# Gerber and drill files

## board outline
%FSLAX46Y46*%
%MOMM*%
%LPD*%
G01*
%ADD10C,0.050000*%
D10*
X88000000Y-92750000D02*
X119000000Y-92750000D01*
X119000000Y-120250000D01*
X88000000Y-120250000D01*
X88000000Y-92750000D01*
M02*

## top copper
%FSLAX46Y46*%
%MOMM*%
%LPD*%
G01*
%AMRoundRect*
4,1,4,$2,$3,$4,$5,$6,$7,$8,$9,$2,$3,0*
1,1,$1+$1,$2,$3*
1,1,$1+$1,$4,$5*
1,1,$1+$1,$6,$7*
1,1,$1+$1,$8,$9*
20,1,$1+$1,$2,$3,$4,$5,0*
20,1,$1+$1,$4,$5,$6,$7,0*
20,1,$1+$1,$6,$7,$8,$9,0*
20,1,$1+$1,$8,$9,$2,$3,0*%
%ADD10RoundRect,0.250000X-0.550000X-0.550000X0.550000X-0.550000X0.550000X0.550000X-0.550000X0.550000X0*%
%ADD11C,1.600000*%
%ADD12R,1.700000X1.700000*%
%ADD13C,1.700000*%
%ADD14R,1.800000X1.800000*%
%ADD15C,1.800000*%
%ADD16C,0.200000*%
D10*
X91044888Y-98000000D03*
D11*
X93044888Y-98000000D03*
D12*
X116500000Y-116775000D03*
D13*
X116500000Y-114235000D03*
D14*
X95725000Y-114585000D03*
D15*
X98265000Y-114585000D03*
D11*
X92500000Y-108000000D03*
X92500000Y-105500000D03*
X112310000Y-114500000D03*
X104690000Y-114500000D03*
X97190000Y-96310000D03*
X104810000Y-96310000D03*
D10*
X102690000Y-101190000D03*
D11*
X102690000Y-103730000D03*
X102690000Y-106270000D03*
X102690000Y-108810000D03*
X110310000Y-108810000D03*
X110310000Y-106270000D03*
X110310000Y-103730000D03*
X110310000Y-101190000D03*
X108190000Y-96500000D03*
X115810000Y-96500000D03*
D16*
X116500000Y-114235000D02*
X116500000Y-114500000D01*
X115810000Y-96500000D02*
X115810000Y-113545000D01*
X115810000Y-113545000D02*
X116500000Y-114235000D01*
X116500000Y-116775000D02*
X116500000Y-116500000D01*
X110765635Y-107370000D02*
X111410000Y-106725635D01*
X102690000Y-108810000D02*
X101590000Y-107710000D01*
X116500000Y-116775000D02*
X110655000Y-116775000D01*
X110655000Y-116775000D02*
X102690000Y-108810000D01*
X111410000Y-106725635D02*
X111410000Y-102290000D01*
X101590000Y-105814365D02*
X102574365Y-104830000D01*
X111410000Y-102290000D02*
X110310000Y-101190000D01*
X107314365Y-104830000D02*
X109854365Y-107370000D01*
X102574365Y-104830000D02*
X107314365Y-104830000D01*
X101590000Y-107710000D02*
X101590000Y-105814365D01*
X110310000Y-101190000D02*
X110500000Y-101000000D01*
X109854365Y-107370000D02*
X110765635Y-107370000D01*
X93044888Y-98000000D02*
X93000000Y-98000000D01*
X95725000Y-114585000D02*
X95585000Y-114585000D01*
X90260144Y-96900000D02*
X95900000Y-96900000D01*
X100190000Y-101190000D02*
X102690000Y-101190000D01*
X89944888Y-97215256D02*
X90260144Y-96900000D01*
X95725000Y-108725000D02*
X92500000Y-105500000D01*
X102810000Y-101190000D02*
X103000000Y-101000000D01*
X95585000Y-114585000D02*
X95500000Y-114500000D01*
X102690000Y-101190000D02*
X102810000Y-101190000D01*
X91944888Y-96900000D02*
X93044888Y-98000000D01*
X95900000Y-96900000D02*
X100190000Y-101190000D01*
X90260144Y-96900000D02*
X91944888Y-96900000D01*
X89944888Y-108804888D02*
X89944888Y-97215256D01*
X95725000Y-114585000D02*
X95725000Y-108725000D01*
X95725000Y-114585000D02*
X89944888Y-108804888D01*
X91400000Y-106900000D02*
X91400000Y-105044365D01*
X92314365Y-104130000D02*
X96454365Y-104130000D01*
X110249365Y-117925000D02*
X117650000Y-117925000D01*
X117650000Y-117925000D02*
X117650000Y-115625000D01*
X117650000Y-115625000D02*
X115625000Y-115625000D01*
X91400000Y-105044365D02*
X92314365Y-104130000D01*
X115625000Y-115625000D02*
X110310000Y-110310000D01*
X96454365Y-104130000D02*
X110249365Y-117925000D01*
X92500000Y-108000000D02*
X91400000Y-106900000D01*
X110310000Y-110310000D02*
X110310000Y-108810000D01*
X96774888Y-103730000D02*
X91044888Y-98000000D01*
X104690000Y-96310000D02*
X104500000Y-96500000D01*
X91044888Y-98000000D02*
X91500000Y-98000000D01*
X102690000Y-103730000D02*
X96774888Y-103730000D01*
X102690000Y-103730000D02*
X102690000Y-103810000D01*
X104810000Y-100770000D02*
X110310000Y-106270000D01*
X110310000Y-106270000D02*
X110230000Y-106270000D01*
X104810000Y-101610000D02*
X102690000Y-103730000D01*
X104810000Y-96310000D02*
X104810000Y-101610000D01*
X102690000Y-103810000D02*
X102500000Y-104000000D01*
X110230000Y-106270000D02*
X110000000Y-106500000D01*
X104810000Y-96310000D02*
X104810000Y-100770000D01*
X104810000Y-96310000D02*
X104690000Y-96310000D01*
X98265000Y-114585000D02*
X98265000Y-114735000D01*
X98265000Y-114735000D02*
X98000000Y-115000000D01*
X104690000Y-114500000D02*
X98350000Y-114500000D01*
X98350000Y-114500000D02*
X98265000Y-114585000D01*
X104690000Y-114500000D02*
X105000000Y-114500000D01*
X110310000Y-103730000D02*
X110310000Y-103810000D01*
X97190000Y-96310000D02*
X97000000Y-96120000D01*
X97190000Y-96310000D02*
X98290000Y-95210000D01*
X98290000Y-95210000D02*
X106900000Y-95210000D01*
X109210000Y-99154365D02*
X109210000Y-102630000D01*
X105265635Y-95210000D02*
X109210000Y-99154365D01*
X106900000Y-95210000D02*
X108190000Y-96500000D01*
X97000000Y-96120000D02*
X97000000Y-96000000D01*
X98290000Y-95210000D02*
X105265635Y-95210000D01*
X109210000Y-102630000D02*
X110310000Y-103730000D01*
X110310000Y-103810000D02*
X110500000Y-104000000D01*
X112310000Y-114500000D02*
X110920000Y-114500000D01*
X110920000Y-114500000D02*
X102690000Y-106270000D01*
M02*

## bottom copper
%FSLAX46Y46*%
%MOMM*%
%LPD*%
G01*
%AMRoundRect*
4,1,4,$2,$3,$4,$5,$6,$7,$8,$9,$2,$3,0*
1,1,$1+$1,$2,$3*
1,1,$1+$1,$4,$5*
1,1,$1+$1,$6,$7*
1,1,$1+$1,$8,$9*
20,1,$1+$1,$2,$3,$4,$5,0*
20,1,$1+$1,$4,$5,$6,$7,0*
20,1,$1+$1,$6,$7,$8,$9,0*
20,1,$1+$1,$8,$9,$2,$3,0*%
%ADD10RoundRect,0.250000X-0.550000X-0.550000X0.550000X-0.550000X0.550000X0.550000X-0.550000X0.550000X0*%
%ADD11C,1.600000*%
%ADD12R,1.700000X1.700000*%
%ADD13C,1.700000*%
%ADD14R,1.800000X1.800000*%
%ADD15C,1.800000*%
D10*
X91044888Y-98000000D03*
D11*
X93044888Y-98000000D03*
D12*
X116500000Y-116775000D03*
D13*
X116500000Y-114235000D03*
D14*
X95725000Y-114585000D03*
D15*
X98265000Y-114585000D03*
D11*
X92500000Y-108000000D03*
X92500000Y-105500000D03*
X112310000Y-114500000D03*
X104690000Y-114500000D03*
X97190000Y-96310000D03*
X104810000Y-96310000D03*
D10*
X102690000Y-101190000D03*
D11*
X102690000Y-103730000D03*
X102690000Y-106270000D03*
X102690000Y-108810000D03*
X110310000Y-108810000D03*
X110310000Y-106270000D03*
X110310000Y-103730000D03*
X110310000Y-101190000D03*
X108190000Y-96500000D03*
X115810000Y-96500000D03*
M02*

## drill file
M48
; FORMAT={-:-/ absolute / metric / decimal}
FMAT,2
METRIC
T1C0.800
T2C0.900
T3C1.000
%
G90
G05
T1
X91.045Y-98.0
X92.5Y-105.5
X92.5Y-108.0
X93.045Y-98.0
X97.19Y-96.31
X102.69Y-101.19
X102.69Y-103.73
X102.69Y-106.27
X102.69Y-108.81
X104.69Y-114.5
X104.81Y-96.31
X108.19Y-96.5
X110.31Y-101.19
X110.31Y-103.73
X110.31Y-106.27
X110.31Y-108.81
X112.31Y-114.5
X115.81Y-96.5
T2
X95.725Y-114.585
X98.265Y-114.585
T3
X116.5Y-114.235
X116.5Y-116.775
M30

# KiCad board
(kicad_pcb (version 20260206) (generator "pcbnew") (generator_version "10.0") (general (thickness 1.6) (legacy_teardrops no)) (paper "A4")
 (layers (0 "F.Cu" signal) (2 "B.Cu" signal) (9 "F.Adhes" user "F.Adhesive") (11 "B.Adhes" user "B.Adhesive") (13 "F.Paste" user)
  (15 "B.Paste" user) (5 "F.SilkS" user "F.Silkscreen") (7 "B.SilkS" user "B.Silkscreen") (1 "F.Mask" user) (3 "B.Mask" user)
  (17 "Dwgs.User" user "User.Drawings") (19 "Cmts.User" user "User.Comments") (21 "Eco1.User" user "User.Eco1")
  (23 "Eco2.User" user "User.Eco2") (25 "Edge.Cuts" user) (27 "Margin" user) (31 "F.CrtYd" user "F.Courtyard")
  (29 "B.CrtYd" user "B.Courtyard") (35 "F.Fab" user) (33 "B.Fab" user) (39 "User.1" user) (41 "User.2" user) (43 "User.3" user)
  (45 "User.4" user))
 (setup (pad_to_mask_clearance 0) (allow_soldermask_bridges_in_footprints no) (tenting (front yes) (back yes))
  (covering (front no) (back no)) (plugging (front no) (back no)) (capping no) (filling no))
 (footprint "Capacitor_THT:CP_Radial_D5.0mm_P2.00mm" (layer "F.Cu") (at 91.044888 98)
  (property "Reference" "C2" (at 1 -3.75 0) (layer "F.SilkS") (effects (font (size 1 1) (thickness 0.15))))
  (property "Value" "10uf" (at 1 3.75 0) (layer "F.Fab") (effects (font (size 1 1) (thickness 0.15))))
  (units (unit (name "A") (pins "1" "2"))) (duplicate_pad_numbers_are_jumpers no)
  (pad "1" thru_hole roundrect (at 0 0) (size 1.6 1.6) (drill 0.8) (layers "*.Cu" "*.Mask") (remove_unused_layers no)
   (roundrect_rratio 0.15625) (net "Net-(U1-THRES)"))
  (pad "2" thru_hole circle (at 2 0) (size 1.6 1.6) (drill 0.8) (layers "*.Cu" "*.Mask") (remove_unused_layers no) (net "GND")))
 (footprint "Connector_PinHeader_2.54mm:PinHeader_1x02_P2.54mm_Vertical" (layer "F.Cu") (at 116.5 116.775 180)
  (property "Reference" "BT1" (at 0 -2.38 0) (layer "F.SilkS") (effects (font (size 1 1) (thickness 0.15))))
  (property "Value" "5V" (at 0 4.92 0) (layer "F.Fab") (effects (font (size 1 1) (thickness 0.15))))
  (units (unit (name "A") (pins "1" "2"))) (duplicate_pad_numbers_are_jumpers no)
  (pad "1" thru_hole rect (at 0 0 180) (size 1.7 1.7) (drill 1) (layers "*.Cu" "*.Mask") (remove_unused_layers no) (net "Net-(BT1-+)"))
  (pad "2" thru_hole circle (at 0 2.54 180) (size 1.7 1.7) (drill 1) (layers "*.Cu" "*.Mask") (remove_unused_layers no) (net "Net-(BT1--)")))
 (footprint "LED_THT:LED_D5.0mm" (layer "F.Cu") (at 95.725 114.585)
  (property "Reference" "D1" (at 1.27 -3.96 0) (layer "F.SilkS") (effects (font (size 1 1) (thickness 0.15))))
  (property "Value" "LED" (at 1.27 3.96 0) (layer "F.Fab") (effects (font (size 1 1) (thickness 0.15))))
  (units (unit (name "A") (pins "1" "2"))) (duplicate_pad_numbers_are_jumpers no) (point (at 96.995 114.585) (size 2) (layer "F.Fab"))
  (pad "1" thru_hole rect (at 0 0) (size 1.8 1.8) (drill 0.9) (layers "*.Cu" "*.Mask") (remove_unused_layers no) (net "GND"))
  (pad "2" thru_hole circle (at 2.54 0) (size 1.8 1.8) (drill 0.9) (layers "*.Cu" "*.Mask") (remove_unused_layers no) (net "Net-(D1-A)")))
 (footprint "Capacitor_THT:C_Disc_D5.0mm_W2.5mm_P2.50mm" (layer "F.Cu") (at 92.5 108 90)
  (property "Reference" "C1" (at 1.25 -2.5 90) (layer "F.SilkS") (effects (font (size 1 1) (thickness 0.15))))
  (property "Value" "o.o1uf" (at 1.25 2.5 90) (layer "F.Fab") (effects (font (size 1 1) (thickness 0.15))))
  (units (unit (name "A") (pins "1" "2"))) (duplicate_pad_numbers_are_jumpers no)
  (pad "1" thru_hole circle (at 0 0 90) (size 1.6 1.6) (drill 0.8) (layers "*.Cu" "*.Mask") (remove_unused_layers no) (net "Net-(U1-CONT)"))
  (pad "2" thru_hole circle (at 2.5 0 90) (size 1.6 1.6) (drill 0.8) (layers "*.Cu" "*.Mask") (remove_unused_layers no) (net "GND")))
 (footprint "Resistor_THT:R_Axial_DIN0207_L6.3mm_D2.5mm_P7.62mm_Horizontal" (layer "F.Cu") (at 112.31 114.5 180)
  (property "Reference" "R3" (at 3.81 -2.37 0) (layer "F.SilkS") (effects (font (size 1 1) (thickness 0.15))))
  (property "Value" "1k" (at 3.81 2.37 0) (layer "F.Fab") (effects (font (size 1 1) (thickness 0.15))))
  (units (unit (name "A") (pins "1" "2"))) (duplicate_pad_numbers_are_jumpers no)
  (pad "1" thru_hole circle (at 0 0 180) (size 1.6 1.6) (drill 0.8) (layers "*.Cu" "*.Mask") (remove_unused_layers no) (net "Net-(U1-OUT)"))
  (pad "2" thru_hole circle (at 7.62 0 180) (size 1.6 1.6) (drill 0.8) (layers "*.Cu" "*.Mask") (remove_unused_layers no) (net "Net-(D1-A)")))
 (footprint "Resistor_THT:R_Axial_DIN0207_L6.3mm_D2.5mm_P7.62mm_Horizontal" (layer "F.Cu") (at 97.19 96.31)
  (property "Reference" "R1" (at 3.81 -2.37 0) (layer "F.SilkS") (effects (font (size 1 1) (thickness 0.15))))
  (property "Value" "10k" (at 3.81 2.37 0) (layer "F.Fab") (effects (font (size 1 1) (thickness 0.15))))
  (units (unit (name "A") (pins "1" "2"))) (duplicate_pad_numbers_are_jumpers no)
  (pad "1" thru_hole circle (at 0 0) (size 1.6 1.6) (drill 0.8) (layers "*.Cu" "*.Mask") (remove_unused_layers no) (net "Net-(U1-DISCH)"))
  (pad "2" thru_hole circle (at 7.62 0) (size 1.6 1.6) (drill 0.8) (layers "*.Cu" "*.Mask") (remove_unused_layers no) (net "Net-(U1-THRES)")))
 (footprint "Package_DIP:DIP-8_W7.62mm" (layer "F.Cu") (at 102.69 101.19)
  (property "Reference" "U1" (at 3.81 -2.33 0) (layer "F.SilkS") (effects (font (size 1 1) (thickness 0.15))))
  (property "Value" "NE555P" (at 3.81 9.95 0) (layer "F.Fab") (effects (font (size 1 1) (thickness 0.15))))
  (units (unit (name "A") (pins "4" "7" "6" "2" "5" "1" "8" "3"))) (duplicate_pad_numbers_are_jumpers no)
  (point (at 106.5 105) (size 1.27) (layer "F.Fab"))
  (pad "1" thru_hole roundrect (at 0 0) (size 1.6 1.6) (drill 0.8) (layers "*.Cu" "*.Mask") (remove_unused_layers no)
   (roundrect_rratio 0.15625) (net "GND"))
  (pad "2" thru_hole circle (at 0 2.54) (size 1.6 1.6) (drill 0.8) (layers "*.Cu" "*.Mask") (remove_unused_layers no) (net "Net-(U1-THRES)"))
  (pad "3" thru_hole circle (at 0 5.08) (size 1.6 1.6) (drill 0.8) (layers "*.Cu" "*.Mask") (remove_unused_layers no) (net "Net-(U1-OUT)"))
  (pad "4" thru_hole circle (at 0 7.62) (size 1.6 1.6) (drill 0.8) (layers "*.Cu" "*.Mask") (remove_unused_layers no) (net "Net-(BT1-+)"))
  (pad "5" thru_hole circle (at 7.62 7.62) (size 1.6 1.6) (drill 0.8) (layers "*.Cu" "*.Mask") (remove_unused_layers no)
   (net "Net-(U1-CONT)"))
  (pad "6" thru_hole circle (at 7.62 5.08) (size 1.6 1.6) (drill 0.8) (layers "*.Cu" "*.Mask") (remove_unused_layers no)
   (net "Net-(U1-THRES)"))
  (pad "7" thru_hole circle (at 7.62 2.54) (size 1.6 1.6) (drill 0.8) (layers "*.Cu" "*.Mask") (remove_unused_layers no)
   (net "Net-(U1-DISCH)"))
  (pad "8" thru_hole circle (at 7.62 0) (size 1.6 1.6) (drill 0.8) (layers "*.Cu" "*.Mask") (remove_unused_layers no) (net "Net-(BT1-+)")))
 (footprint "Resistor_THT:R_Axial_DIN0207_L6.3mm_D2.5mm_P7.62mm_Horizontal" (layer "F.Cu") (at 108.19 96.5)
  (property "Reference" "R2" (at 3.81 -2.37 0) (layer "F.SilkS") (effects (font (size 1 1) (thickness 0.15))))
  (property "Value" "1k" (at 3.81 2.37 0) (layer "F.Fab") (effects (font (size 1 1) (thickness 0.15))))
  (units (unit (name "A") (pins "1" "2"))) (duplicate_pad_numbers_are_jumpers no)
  (pad "1" thru_hole circle (at 0 0) (size 1.6 1.6) (drill 0.8) (layers "*.Cu" "*.Mask") (remove_unused_layers no) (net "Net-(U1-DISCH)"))
  (pad "2" thru_hole circle (at 7.62 0) (size 1.6 1.6) (drill 0.8) (layers "*.Cu" "*.Mask") (remove_unused_layers no) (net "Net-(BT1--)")))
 (gr_rect (start 88 92.75) (end 119 120.25) (stroke (width 0.05) (type default)) (fill no) (layer "Edge.Cuts"))
 (segment (start 116.5 114.235) (end 116.5 114.5) (width 0.2) (layer "F.Cu") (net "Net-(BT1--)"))
 (segment (start 115.81 96.5) (end 115.81 113.545) (width 0.2) (layer "F.Cu") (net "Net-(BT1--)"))
 (segment (start 115.81 113.545) (end 116.5 114.235) (width 0.2) (layer "F.Cu") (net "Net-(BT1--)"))
 (segment (start 116.5 116.775) (end 116.5 116.5) (width 0.2) (layer "F.Cu") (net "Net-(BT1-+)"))
 (segment (start 110.765635 107.37) (end 111.41 106.725635) (width 0.2) (layer "F.Cu") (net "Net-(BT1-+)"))
 (segment (start 102.69 108.81) (end 101.59 107.71) (width 0.2) (layer "F.Cu") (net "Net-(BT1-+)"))
 (segment (start 116.5 116.775) (end 110.655 116.775) (width 0.2) (layer "F.Cu") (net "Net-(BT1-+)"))
 (segment (start 110.655 116.775) (end 102.69 108.81) (width 0.2) (layer "F.Cu") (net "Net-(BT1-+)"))
 (segment (start 111.41 106.725635) (end 111.41 102.29) (width 0.2) (layer "F.Cu") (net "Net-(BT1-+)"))
 (segment (start 101.59 105.814365) (end 102.574365 104.83) (width 0.2) (layer "F.Cu") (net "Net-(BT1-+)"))
 (segment (start 111.41 102.29) (end 110.31 101.19) (width 0.2) (layer "F.Cu") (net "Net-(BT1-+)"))
 (segment (start 107.314365 104.83) (end 109.854365 107.37) (width 0.2) (layer "F.Cu") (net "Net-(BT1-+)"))
 (segment (start 102.574365 104.83) (end 107.314365 104.83) (width 0.2) (layer "F.Cu") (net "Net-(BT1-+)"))
 (segment (start 101.59 107.71) (end 101.59 105.814365) (width 0.2) (layer "F.Cu") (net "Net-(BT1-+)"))
 (segment (start 110.31 101.19) (end 110.5 101) (width 0.2) (layer "F.Cu") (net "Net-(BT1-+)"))
 (segment (start 109.854365 107.37) (end 110.765635 107.37) (width 0.2) (layer "F.Cu") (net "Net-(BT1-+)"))
 (segment (start 93.044888 98) (end 93 98) (width 0.2) (layer "F.Cu") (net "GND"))
 (segment (start 95.725 114.585) (end 95.585 114.585) (width 0.2) (layer "F.Cu") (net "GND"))
 (segment (start 90.260144 96.9) (end 95.9 96.9) (width 0.2) (layer "F.Cu") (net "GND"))
 (segment (start 100.19 101.19) (end 102.69 101.19) (width 0.2) (layer "F.Cu") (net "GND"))
 (segment (start 89.944888 97.215256) (end 90.260144 96.9) (width 0.2) (layer "F.Cu") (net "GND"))
 (segment (start 95.725 108.725) (end 92.5 105.5) (width 0.2) (layer "F.Cu") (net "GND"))
 (segment (start 102.81 101.19) (end 103 101) (width 0.2) (layer "F.Cu") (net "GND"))
 (segment (start 95.585 114.585) (end 95.5 114.5) (width 0.2) (layer "F.Cu") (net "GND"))
 (segment (start 102.69 101.19) (end 102.81 101.19) (width 0.2) (layer "F.Cu") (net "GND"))
 (segment (start 91.944888 96.9) (end 93.044888 98) (width 0.2) (layer "F.Cu") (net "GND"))
 (segment (start 95.9 96.9) (end 100.19 101.19) (width 0.2) (layer "F.Cu") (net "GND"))
 (segment (start 90.260144 96.9) (end 91.944888 96.9) (width 0.2) (layer "F.Cu") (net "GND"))
 (segment (start 89.944888 108.804888) (end 89.944888 97.215256) (width 0.2) (layer "F.Cu") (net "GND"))
 (segment (start 95.725 114.585) (end 95.725 108.725) (width 0.2) (layer "F.Cu") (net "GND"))
 (segment (start 95.725 114.585) (end 89.944888 108.804888) (width 0.2) (layer "F.Cu") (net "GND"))
 (segment (start 91.4 106.9) (end 91.4 105.044365) (width 0.2) (layer "F.Cu") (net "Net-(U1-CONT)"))
 (segment (start 92.314365 104.13) (end 96.454365 104.13) (width 0.2) (layer "F.Cu") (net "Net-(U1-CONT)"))
 (segment (start 110.249365 117.925) (end 117.65 117.925) (width 0.2) (layer "F.Cu") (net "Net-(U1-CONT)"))
 (segment (start 117.65 117.925) (end 117.65 115.625) (width 0.2) (layer "F.Cu") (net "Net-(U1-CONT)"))
 (segment (start 117.65 115.625) (end 115.625 115.625) (width 0.2) (layer "F.Cu") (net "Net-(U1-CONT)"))
 (segment (start 91.4 105.044365) (end 92.314365 104.13) (width 0.2) (layer "F.Cu") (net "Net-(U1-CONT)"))
 (segment (start 115.625 115.625) (end 110.31 110.31) (width 0.2) (layer "F.Cu") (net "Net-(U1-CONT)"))
 (segment (start 96.454365 104.13) (end 110.249365 117.925) (width 0.2) (layer "F.Cu") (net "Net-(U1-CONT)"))
 (segment (start 92.5 108) (end 91.4 106.9) (width 0.2) (layer "F.Cu") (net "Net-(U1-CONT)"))
 (segment (start 110.31 110.31) (end 110.31 108.81) (width 0.2) (layer "F.Cu") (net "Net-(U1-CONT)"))
 (segment (start 96.774888 103.73) (end 91.044888 98) (width 0.2) (layer "F.Cu") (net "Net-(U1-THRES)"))
 (segment (start 104.69 96.31) (end 104.5 96.5) (width 0.2) (layer "F.Cu") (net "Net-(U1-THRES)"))
 (segment (start 91.044888 98) (end 91.5 98) (width 0.2) (layer "F.Cu") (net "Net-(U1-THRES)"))
 (segment (start 102.69 103.73) (end 96.774888 103.73) (width 0.2) (layer "F.Cu") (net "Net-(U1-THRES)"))
 (segment (start 102.69 103.73) (end 102.69 103.81) (width 0.2) (layer "F.Cu") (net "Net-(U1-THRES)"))
 (segment (start 104.81 100.77) (end 110.31 106.27) (width 0.2) (layer "F.Cu") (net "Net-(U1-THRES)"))
 (segment (start 110.31 106.27) (end 110.23 106.27) (width 0.2) (layer "F.Cu") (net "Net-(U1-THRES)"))
 (segment (start 104.81 101.61) (end 102.69 103.73) (width 0.2) (layer "F.Cu") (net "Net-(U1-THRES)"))
 (segment (start 104.81 96.31) (end 104.81 101.61) (width 0.2) (layer "F.Cu") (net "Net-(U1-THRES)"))
 (segment (start 102.69 103.81) (end 102.5 104) (width 0.2) (layer "F.Cu") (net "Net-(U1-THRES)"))
 (segment (start 110.23 106.27) (end 110 106.5) (width 0.2) (layer "F.Cu") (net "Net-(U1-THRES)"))
 (segment (start 104.81 96.31) (end 104.81 100.77) (width 0.2) (layer "F.Cu") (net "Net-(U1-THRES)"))
 (segment (start 104.81 96.31) (end 104.69 96.31) (width 0.2) (layer "F.Cu") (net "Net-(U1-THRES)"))
 (segment (start 98.265 114.585) (end 98.265 114.735) (width 0.2) (layer "F.Cu") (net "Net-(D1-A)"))
 (segment (start 98.265 114.735) (end 98 115) (width 0.2) (layer "F.Cu") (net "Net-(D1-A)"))
 (segment (start 104.69 114.5) (end 98.35 114.5) (width 0.2) (layer "F.Cu") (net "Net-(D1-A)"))
 (segment (start 98.35 114.5) (end 98.265 114.585) (width 0.2) (layer "F.Cu") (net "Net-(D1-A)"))
 (segment (start 104.69 114.5) (end 105 114.5) (width 0.2) (layer "F.Cu") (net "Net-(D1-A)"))
 (segment (start 110.31 103.73) (end 110.31 103.81) (width 0.2) (layer "F.Cu") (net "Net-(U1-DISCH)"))
 (segment (start 97.19 96.31) (end 97 96.12) (width 0.2) (layer "F.Cu") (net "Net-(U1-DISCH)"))
 (segment (start 97.19 96.31) (end 98.29 95.21) (width 0.2) (layer "F.Cu") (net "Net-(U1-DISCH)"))
 (segment (start 98.29 95.21) (end 106.9 95.21) (width 0.2) (layer "F.Cu") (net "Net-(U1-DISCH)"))
 (segment (start 109.21 99.154365) (end 109.21 102.63) (width 0.2) (layer "F.Cu") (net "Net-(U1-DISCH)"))
 (segment (start 105.265635 95.21) (end 109.21 99.154365) (width 0.2) (layer "F.Cu") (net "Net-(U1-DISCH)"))
 (segment (start 106.9 95.21) (end 108.19 96.5) (width 0.2) (layer "F.Cu") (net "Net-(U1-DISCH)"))
 (segment (start 97 96.12) (end 97 96) (width 0.2) (layer "F.Cu") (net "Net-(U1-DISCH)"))
 (segment (start 98.29 95.21) (end 105.265635 95.21) (width 0.2) (layer "F.Cu") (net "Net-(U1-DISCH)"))
 (segment (start 109.21 102.63) (end 110.31 103.73) (width 0.2) (layer "F.Cu") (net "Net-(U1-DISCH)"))
 (segment (start 110.31 103.81) (end 110.5 104) (width 0.2) (layer "F.Cu") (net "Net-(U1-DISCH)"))
 (segment (start 112.31 114.5) (end 110.92 114.5) (width 0.2) (layer "F.Cu") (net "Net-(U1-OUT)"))
 (segment (start 110.92 114.5) (end 102.69 106.27) (width 0.2) (layer "F.Cu") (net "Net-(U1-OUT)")))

